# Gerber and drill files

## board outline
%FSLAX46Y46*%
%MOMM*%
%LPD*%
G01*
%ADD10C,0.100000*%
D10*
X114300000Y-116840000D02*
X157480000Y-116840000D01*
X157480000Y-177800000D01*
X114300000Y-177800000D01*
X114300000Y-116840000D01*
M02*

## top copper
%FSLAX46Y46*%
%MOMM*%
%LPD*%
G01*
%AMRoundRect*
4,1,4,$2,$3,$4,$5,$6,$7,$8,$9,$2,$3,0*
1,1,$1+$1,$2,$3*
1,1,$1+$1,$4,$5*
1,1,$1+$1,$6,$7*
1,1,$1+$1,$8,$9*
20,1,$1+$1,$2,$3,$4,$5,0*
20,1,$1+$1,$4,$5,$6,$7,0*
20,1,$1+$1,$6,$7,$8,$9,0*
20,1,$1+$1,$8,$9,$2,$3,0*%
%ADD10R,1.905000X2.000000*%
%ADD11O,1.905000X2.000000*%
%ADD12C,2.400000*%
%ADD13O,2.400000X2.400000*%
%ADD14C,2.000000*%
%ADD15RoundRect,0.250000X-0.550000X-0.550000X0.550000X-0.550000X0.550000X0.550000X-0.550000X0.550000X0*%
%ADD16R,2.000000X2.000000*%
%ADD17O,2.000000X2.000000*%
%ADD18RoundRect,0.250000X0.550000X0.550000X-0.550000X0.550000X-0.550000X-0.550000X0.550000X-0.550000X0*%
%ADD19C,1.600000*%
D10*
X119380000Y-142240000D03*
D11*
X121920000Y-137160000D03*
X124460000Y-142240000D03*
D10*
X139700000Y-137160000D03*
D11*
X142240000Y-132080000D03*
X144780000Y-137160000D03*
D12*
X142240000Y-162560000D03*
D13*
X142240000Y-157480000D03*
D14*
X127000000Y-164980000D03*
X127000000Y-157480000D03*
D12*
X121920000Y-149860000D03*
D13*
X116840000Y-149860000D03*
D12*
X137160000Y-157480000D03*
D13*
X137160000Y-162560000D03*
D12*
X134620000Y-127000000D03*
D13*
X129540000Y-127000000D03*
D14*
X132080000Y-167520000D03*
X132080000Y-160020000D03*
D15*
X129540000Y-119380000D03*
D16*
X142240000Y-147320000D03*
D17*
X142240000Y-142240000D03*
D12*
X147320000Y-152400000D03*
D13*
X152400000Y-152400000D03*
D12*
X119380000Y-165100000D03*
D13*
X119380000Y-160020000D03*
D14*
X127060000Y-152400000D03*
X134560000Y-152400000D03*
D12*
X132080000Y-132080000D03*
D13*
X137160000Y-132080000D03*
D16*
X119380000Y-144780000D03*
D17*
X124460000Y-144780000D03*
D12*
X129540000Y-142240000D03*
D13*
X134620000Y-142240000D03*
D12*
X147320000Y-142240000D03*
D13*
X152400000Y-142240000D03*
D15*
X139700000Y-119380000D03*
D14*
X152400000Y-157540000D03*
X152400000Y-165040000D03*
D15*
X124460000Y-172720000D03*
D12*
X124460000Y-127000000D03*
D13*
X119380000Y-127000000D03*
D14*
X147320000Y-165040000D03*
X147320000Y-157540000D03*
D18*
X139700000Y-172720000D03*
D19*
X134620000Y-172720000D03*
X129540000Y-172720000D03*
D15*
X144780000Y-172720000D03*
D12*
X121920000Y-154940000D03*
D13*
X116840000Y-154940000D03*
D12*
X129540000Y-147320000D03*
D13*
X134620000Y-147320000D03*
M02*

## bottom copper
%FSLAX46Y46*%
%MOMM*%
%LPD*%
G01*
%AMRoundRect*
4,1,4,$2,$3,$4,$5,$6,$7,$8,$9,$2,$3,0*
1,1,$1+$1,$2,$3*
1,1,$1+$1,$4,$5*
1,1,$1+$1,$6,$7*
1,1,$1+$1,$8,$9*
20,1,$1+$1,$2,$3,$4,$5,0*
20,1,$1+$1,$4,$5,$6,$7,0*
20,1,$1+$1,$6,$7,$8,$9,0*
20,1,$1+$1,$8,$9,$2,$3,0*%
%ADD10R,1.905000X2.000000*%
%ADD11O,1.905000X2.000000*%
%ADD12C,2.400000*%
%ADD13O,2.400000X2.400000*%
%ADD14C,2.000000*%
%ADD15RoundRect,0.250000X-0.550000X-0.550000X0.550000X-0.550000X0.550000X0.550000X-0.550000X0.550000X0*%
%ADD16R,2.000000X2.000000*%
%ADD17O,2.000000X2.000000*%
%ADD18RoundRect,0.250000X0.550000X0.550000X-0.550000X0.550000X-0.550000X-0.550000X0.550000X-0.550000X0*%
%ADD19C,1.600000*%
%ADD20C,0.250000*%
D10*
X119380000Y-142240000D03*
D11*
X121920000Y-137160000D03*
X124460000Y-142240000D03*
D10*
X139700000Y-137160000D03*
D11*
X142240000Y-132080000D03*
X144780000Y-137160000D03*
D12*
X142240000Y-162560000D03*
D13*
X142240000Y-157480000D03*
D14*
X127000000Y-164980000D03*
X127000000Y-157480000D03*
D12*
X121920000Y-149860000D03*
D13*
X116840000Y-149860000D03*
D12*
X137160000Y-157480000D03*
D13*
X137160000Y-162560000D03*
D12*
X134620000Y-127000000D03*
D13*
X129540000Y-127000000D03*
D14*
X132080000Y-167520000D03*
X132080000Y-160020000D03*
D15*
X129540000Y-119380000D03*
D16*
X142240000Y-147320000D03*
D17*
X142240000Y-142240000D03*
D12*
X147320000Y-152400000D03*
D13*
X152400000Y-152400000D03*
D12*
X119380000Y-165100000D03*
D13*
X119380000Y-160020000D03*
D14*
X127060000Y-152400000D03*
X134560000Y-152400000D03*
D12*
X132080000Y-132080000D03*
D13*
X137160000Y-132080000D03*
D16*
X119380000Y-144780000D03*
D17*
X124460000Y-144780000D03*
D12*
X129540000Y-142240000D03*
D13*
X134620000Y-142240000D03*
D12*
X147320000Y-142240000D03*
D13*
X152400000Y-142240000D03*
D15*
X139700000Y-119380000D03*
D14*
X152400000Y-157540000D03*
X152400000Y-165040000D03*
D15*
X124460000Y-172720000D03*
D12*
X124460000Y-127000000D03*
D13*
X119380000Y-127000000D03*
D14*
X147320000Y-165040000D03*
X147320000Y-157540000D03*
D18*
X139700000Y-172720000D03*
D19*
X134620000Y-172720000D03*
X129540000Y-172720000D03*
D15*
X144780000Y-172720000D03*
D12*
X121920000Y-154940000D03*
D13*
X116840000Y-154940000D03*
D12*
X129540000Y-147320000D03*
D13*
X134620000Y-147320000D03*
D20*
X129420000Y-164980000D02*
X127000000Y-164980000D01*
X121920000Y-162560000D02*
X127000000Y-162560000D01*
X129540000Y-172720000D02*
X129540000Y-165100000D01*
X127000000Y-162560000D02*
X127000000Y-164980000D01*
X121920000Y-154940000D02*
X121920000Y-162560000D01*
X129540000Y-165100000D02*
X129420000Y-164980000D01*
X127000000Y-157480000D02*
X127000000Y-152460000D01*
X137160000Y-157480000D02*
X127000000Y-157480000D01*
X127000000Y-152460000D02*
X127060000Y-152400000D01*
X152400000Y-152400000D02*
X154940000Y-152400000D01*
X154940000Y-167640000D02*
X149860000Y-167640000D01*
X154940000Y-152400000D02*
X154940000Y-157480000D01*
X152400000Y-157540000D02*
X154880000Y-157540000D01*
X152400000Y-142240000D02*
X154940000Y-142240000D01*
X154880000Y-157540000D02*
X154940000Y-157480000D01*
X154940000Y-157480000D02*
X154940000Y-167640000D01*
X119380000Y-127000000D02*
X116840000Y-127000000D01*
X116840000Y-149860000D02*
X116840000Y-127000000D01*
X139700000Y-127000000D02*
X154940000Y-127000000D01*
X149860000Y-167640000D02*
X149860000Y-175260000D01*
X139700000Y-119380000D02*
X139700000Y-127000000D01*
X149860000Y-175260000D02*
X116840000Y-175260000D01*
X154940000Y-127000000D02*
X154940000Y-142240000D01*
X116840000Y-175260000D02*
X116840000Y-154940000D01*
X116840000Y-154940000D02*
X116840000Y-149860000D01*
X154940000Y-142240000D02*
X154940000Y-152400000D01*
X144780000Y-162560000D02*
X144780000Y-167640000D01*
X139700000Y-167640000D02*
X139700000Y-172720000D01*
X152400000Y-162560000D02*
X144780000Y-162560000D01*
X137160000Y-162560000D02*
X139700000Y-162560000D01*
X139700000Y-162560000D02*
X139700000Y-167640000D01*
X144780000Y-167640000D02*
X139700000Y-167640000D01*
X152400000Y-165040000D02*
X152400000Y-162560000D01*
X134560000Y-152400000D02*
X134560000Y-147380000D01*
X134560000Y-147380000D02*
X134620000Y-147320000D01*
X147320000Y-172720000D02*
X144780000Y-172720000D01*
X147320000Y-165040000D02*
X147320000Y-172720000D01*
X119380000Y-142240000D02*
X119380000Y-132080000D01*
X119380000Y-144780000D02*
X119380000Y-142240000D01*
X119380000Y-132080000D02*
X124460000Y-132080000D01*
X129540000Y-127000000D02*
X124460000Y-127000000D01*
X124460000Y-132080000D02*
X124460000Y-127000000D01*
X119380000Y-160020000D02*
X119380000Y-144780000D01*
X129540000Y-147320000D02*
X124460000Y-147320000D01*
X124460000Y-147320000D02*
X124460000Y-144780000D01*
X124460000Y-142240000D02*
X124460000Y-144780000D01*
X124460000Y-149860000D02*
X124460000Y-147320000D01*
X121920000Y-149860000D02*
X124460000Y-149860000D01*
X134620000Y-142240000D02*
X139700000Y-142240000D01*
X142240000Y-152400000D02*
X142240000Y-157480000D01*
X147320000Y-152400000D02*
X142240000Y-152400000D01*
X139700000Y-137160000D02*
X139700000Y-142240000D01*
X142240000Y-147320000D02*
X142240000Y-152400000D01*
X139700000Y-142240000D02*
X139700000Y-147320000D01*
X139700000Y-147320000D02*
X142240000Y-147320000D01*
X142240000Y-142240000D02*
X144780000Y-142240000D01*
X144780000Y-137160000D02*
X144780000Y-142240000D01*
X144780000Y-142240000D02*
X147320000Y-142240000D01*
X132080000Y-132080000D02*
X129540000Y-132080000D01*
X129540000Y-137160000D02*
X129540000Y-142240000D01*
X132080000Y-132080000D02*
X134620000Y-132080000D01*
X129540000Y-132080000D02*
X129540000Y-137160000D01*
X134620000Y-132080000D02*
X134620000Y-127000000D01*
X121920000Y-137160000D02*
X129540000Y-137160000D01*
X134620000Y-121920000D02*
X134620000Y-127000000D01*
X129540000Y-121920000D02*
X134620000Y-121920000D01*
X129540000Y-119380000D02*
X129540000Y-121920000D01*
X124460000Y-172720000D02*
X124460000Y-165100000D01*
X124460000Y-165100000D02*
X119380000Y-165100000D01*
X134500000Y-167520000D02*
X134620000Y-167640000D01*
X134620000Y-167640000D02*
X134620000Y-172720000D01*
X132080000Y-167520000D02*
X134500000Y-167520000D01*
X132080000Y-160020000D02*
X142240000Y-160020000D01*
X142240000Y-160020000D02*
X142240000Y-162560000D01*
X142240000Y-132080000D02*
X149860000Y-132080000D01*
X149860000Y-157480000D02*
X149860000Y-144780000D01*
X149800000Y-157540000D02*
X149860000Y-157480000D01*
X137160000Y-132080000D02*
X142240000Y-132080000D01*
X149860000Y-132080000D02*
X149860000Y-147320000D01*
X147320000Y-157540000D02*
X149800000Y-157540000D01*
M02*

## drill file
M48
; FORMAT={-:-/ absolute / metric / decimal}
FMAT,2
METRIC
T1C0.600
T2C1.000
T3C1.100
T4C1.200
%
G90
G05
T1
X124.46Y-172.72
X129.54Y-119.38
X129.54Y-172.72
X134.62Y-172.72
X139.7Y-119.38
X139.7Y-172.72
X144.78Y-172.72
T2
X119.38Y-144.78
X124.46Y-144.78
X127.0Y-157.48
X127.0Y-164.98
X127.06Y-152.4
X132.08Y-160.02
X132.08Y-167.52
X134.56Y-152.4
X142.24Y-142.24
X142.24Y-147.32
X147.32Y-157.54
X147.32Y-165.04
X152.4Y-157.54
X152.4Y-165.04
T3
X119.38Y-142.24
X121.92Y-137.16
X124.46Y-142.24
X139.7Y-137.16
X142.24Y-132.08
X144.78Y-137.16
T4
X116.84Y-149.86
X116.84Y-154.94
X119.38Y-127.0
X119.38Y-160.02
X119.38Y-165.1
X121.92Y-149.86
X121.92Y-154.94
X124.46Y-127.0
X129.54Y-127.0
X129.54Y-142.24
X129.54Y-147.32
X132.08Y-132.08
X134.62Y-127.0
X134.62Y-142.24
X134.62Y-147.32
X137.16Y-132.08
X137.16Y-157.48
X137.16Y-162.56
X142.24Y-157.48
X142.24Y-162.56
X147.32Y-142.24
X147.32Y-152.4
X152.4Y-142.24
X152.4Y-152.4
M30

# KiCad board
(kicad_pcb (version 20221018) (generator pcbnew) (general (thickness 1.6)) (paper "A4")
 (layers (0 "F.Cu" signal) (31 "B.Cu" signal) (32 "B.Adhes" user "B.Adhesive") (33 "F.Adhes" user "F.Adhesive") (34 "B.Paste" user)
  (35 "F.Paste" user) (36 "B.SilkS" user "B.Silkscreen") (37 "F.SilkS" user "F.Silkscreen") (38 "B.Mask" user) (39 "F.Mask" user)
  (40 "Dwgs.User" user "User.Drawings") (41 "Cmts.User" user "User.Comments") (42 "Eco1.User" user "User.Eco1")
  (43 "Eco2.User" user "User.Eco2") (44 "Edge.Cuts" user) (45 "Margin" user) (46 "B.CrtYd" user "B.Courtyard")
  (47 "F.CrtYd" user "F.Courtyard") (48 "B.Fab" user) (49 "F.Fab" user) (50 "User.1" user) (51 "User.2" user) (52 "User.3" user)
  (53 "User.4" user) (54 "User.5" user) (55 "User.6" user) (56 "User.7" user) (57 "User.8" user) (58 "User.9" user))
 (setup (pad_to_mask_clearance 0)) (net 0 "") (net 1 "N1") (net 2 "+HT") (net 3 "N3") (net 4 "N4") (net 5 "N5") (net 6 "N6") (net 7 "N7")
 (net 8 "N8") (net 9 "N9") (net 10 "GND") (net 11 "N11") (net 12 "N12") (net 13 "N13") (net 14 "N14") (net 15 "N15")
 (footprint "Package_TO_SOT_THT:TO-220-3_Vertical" (layer "F.Cu") (at 119.38 137.16)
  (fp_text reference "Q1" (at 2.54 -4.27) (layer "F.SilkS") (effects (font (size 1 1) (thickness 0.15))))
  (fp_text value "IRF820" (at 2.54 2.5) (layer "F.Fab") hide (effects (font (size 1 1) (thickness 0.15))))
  (pad "1" thru_hole rect (at 0 5.08) (size 1.905 2) (drill 1.1) (layers "*.Cu" "*.Mask") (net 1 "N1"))
  (pad "2" thru_hole oval (at 2.54 0) (size 1.905 2) (drill 1.1) (layers "*.Cu" "*.Mask") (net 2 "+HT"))
  (pad "3" thru_hole oval (at 5.08 5.08) (size 1.905 2) (drill 1.1) (layers "*.Cu" "*.Mask") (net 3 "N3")))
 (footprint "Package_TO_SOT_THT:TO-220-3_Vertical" (layer "F.Cu") (at 139.7 137.16)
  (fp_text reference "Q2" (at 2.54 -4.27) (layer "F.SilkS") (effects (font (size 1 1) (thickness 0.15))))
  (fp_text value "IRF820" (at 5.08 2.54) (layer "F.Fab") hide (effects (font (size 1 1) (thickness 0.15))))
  (pad "1" thru_hole rect (at 0 0) (size 1.905 2) (drill 1.1) (layers "*.Cu" "*.Mask") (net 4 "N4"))
  (pad "2" thru_hole oval (at 2.54 -5.08) (size 1.905 2) (drill 1.1) (layers "*.Cu" "*.Mask") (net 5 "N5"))
  (pad "3" thru_hole oval (at 5.08 0) (size 1.905 2) (drill 1.1) (layers "*.Cu" "*.Mask") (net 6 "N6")))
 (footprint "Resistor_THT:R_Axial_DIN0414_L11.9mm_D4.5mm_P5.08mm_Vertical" (layer "F.Cu") (at 142.24 162.56 90)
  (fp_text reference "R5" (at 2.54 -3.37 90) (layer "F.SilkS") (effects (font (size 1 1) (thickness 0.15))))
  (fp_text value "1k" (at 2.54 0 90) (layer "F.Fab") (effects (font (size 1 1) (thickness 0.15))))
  (pad "1" thru_hole circle (at 0 0 90) (size 2.4 2.4) (drill 1.2) (layers "*.Cu" "*.Mask") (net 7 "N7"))
  (pad "2" thru_hole oval (at 5.08 0 90) (size 2.4 2.4) (drill 1.2) (layers "*.Cu" "*.Mask") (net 4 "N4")))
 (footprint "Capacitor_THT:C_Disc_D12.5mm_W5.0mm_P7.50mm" (layer "F.Cu") (at 127 164.98 90)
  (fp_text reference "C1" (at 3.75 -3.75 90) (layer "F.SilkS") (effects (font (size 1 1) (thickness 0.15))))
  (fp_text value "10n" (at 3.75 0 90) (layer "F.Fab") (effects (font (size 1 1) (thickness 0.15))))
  (pad "1" thru_hole circle (at 0 0 90) (size 2 2) (drill 1) (layers "*.Cu" "*.Mask") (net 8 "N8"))
  (pad "2" thru_hole circle (at 7.5 0 90) (size 2 2) (drill 1) (layers "*.Cu" "*.Mask") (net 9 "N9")))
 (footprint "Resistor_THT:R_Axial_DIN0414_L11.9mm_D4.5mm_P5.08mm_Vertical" (layer "F.Cu") (at 121.92 149.86 180)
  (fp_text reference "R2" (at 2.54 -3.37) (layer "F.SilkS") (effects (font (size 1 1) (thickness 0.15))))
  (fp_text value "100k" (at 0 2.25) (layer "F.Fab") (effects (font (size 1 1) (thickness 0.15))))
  (pad "1" thru_hole circle (at 0 0 180) (size 2.4 2.4) (drill 1.2) (layers "*.Cu" "*.Mask") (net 3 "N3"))
  (pad "2" thru_hole oval (at 5.08 0 180) (size 2.4 2.4) (drill 1.2) (layers "*.Cu" "*.Mask") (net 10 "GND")))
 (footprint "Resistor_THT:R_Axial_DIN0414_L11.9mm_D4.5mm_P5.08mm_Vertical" (layer "F.Cu") (at 137.16 157.48 -90)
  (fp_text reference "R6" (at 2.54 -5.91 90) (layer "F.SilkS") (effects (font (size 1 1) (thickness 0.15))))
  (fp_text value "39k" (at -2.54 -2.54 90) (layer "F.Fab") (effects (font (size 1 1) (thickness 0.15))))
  (pad "1" thru_hole circle (at 0 0 270) (size 2.4 2.4) (drill 1.2) (layers "*.Cu" "*.Mask") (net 9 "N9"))
  (pad "2" thru_hole oval (at 5.08 0 270) (size 2.4 2.4) (drill 1.2) (layers "*.Cu" "*.Mask") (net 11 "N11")))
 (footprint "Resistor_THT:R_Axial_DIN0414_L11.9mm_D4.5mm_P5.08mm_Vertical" (layer "F.Cu") (at 134.62 127 180)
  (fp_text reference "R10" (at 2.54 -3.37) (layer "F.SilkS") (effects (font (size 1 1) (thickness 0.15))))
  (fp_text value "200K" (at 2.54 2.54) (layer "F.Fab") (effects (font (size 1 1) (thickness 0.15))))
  (pad "1" thru_hole circle (at 0 0 180) (size 2.4 2.4) (drill 1.2) (layers "*.Cu" "*.Mask") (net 2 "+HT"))
  (pad "2" thru_hole oval (at 5.08 0 180) (size 2.4 2.4) (drill 1.2) (layers "*.Cu" "*.Mask") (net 1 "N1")))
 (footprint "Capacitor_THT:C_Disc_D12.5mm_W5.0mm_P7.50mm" (layer "F.Cu") (at 132.08 167.52 90)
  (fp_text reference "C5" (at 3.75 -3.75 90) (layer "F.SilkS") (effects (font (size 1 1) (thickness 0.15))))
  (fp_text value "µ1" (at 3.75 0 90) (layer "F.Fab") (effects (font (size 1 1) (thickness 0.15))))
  (pad "1" thru_hole circle (at 0 0 90) (size 2 2) (drill 1) (layers "*.Cu" "*.Mask") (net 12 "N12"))
  (pad "2" thru_hole circle (at 7.5 0 90) (size 2 2) (drill 1) (layers "*.Cu" "*.Mask") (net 7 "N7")))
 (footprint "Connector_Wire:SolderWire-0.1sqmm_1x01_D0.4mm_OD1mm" (layer "F.Cu") (at 129.54 119.38)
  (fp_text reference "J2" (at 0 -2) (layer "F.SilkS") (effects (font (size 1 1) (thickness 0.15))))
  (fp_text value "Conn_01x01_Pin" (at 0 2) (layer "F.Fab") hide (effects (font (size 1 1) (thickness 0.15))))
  (pad "1" thru_hole roundrect (at 0 0) (size 1.6 1.6) (drill 0.6) (layers "*.Cu" "*.Mask") (roundrect_rratio 0.15625) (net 2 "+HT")))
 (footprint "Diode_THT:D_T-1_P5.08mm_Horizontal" (layer "F.Cu") (at 142.24 147.32 90)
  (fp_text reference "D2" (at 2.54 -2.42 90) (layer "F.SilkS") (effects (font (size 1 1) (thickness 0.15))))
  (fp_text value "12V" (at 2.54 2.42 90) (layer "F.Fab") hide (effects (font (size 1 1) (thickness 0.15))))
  (pad "1" thru_hole rect (at 0 0 90) (size 2 2) (drill 1) (layers "*.Cu" "*.Mask") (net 4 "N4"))
  (pad "2" thru_hole oval (at 5.08 0 90) (size 2 2) (drill 1) (layers "*.Cu" "*.Mask") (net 6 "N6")))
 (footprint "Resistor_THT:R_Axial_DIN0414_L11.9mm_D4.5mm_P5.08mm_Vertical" (layer "F.Cu") (at 147.32 152.4)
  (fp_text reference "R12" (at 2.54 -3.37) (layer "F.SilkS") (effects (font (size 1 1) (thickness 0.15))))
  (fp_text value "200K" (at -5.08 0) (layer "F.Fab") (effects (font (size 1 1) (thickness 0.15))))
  (pad "1" thru_hole circle (at 0 0) (size 2.4 2.4) (drill 1.2) (layers "*.Cu" "*.Mask") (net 4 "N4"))
  (pad "2" thru_hole oval (at 5.08 0) (size 2.4 2.4) (drill 1.2) (layers "*.Cu" "*.Mask") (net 10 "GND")))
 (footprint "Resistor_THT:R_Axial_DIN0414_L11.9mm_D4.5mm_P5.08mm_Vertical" (layer "F.Cu") (at 119.38 165.1 90)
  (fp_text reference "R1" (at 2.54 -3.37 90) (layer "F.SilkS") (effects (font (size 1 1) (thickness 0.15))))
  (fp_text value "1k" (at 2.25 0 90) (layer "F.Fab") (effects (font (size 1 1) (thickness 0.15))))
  (pad "1" thru_hole circle (at 0 0 90) (size 2.4 2.4) (drill 1.2) (layers "*.Cu" "*.Mask") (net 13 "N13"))
  (pad "2" thru_hole oval (at 5.08 0 90) (size 2.4 2.4) (drill 1.2) (layers "*.Cu" "*.Mask") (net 1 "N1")))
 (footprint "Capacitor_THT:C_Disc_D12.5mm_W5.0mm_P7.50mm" (layer "F.Cu") (at 127.06 152.4)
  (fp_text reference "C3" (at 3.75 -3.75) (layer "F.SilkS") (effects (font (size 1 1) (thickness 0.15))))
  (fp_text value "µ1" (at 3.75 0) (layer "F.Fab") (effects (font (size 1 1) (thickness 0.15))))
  (pad "1" thru_hole circle (at 0 0) (size 2 2) (drill 1) (layers "*.Cu" "*.Mask") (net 9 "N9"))
  (pad "2" thru_hole circle (at 7.5 0) (size 2 2) (drill 1) (layers "*.Cu" "*.Mask") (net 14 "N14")))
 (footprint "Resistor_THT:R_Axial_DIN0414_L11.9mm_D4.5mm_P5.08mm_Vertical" (layer "F.Cu") (at 132.08 132.08)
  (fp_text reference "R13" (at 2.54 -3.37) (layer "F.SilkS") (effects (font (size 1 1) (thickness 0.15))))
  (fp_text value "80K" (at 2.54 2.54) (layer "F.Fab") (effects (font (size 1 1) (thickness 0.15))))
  (pad "1" thru_hole circle (at 0 0) (size 2.4 2.4) (drill 1.2) (layers "*.Cu" "*.Mask") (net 2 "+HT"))
  (pad "2" thru_hole oval (at 5.08 0) (size 2.4 2.4) (drill 1.2) (layers "*.Cu" "*.Mask") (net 5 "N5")))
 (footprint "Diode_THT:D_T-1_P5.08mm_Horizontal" (layer "F.Cu") (at 119.38 144.78)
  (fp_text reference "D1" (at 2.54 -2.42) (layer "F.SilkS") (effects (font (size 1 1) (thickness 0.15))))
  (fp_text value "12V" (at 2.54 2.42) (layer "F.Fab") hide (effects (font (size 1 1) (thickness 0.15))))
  (pad "1" thru_hole rect (at 0 0) (size 2 2) (drill 1) (layers "*.Cu" "*.Mask") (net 1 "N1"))
  (pad "2" thru_hole oval (at 5.08 0) (size 2 2) (drill 1) (layers "*.Cu" "*.Mask") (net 3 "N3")))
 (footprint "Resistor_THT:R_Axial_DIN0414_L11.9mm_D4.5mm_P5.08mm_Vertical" (layer "F.Cu") (at 129.54 142.24)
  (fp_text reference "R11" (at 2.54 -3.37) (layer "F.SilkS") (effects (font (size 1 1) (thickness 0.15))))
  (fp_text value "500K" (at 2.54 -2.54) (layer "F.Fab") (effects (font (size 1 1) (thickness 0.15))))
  (pad "1" thru_hole circle (at 0 0) (size 2.4 2.4) (drill 1.2) (layers "*.Cu" "*.Mask") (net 2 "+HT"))
  (pad "2" thru_hole oval (at 5.08 0) (size 2.4 2.4) (drill 1.2) (layers "*.Cu" "*.Mask") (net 4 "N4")))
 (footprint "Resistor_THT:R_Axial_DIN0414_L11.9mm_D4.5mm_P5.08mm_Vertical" (layer "F.Cu") (at 147.32 142.24)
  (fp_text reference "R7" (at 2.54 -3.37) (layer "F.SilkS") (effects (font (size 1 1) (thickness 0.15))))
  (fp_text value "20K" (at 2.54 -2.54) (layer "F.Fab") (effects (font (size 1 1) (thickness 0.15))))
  (pad "1" thru_hole circle (at 0 0) (size 2.4 2.4) (drill 1.2) (layers "*.Cu" "*.Mask") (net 6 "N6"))
  (pad "2" thru_hole oval (at 5.08 0) (size 2.4 2.4) (drill 1.2) (layers "*.Cu" "*.Mask") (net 10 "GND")))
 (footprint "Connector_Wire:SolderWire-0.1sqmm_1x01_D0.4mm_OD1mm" (layer "F.Cu") (at 139.7 119.38)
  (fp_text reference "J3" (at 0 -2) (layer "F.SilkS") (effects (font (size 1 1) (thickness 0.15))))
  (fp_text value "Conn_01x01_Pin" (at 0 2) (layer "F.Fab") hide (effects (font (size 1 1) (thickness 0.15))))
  (pad "1" thru_hole roundrect (at 0 0) (size 1.6 1.6) (drill 0.6) (layers "*.Cu" "*.Mask") (roundrect_rratio 0.15625) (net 10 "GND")))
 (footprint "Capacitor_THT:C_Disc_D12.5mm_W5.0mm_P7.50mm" (layer "F.Cu") (at 152.4 157.54 -90)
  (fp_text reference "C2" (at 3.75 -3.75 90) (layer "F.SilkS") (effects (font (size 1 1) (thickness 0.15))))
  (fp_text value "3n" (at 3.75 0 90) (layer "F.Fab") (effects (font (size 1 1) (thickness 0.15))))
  (pad "1" thru_hole circle (at 0 0 270) (size 2 2) (drill 1) (layers "*.Cu" "*.Mask") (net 10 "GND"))
  (pad "2" thru_hole circle (at 7.5 0 270) (size 2 2) (drill 1) (layers "*.Cu" "*.Mask") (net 11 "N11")))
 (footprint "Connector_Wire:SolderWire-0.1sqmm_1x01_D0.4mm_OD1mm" (layer "F.Cu") (at 124.46 172.72)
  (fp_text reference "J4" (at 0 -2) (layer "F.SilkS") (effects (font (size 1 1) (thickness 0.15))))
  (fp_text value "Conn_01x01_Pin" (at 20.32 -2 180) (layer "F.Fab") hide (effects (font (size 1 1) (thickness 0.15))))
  (pad "1" thru_hole roundrect (at 0 0) (size 1.6 1.6) (drill 0.6) (layers "*.Cu" "*.Mask") (roundrect_rratio 0.15625) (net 13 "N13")))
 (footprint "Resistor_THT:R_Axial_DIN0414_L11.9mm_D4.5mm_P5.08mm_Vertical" (layer "F.Cu") (at 124.46 127 180)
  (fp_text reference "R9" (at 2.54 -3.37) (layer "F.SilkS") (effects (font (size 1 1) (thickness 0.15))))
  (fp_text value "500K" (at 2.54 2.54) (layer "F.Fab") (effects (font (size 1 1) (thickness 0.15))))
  (pad "1" thru_hole circle (at 0 0 180) (size 2.4 2.4) (drill 1.2) (layers "*.Cu" "*.Mask") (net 1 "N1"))
  (pad "2" thru_hole oval (at 5.08 0 180) (size 2.4 2.4) (drill 1.2) (layers "*.Cu" "*.Mask") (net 10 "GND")))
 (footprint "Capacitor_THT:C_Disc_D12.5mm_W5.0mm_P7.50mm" (layer "F.Cu") (at 147.32 165.04 90)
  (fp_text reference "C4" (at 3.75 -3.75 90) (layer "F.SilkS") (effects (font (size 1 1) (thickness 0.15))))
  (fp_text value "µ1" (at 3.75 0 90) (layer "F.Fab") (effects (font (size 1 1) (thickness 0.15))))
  (pad "1" thru_hole circle (at 0 0 90) (size 2 2) (drill 1) (layers "*.Cu" "*.Mask") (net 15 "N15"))
  (pad "2" thru_hole circle (at 7.5 0 90) (size 2 2) (drill 1) (layers "*.Cu" "*.Mask") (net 5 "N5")))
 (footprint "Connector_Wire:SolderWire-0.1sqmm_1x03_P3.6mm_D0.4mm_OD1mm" (layer "F.Cu") (at 139.7 172.72 180)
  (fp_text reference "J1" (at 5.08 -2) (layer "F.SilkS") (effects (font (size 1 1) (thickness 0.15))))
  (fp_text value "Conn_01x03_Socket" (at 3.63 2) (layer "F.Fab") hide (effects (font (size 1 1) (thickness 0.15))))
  (pad "1" thru_hole roundrect (at 0 0 180) (size 1.6 1.6) (drill 0.6) (layers "*.Cu" "*.Mask") (roundrect_rratio 0.15625) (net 11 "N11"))
  (pad "2" thru_hole circle (at 5.08 0 180) (size 1.6 1.6) (drill 0.6) (layers "*.Cu" "*.Mask") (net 12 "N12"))
  (pad "3" thru_hole circle (at 10.16 0 180) (size 1.6 1.6) (drill 0.6) (layers "*.Cu" "*.Mask") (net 8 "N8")))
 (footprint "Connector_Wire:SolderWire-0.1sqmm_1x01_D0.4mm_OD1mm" (layer "F.Cu") (at 144.78 172.72)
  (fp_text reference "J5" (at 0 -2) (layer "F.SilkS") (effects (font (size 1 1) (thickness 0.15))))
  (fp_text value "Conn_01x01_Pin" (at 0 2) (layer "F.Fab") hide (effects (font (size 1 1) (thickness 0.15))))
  (pad "1" thru_hole roundrect (at 0 0) (size 1.6 1.6) (drill 0.6) (layers "*.Cu" "*.Mask") (roundrect_rratio 0.15625) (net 15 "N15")))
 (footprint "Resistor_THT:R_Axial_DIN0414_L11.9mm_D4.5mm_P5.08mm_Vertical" (layer "F.Cu") (at 121.92 154.94 180)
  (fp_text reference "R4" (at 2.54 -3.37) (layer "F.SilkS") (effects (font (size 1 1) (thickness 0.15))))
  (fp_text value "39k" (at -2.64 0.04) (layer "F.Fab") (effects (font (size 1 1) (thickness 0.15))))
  (pad "1" thru_hole circle (at 0 0 180) (size 2.4 2.4) (drill 1.2) (layers "*.Cu" "*.Mask") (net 8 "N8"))
  (pad "2" thru_hole oval (at 5.08 0 180) (size 2.4 2.4) (drill 1.2) (layers "*.Cu" "*.Mask") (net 10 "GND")))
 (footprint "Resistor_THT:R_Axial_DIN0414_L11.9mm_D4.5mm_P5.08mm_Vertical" (layer "F.Cu") (at 129.54 147.32)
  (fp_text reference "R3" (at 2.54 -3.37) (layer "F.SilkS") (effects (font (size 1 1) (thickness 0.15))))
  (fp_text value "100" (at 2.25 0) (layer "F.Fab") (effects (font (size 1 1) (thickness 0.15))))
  (pad "1" thru_hole circle (at 0 0) (size 2.4 2.4) (drill 1.2) (layers "*.Cu" "*.Mask") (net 3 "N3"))
  (pad "2" thru_hole oval (at 5.08 0) (size 2.4 2.4) (drill 1.2) (layers "*.Cu" "*.Mask") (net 14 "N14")))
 (gr_rect (start 114.3 116.84) (end 157.48 177.8) (stroke (width 0.1) (type default)) (fill none) (layer "Edge.Cuts"))
 (segment (start 129.42 164.98) (end 127 164.98) (width 0.25) (layer "B.Cu") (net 8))
 (segment (start 121.92 162.56) (end 127 162.56) (width 0.25) (layer "B.Cu") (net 8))
 (segment (start 129.54 172.72) (end 129.54 165.1) (width 0.25) (layer "B.Cu") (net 8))
 (segment (start 127 162.56) (end 127 164.98) (width 0.25) (layer "B.Cu") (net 8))
 (segment (start 121.92 154.94) (end 121.92 162.56) (width 0.25) (layer "B.Cu") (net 8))
 (segment (start 129.54 165.1) (end 129.42 164.98) (width 0.25) (layer "B.Cu") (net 8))
 (segment (start 127 157.48) (end 127 152.46) (width 0.25) (layer "B.Cu") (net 9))
 (segment (start 137.16 157.48) (end 127 157.48) (width 0.25) (layer "B.Cu") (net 9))
 (segment (start 127 152.46) (end 127.06 152.4) (width 0.25) (layer "B.Cu") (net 9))
 (segment (start 152.4 152.4) (end 154.94 152.4) (width 0.25) (layer "B.Cu") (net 10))
 (segment (start 154.94 167.64) (end 149.86 167.64) (width 0.25) (layer "B.Cu") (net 10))
 (segment (start 154.94 152.4) (end 154.94 157.48) (width 0.25) (layer "B.Cu") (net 10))
 (segment (start 152.4 157.54) (end 154.88 157.54) (width 0.25) (layer "B.Cu") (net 10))
 (segment (start 152.4 142.24) (end 154.94 142.24) (width 0.25) (layer "B.Cu") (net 10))
 (segment (start 154.88 157.54) (end 154.94 157.48) (width 0.25) (layer "B.Cu") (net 10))
 (segment (start 154.94 157.48) (end 154.94 167.64) (width 0.25) (layer "B.Cu") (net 10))
 (segment (start 119.38 127) (end 116.84 127) (width 0.25) (layer "B.Cu") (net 10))
 (segment (start 116.84 149.86) (end 116.84 127) (width 0.25) (layer "B.Cu") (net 10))
 (segment (start 139.7 127) (end 154.94 127) (width 0.25) (layer "B.Cu") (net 10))
 (segment (start 149.86 167.64) (end 149.86 175.26) (width 0.25) (layer "B.Cu") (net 10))
 (segment (start 139.7 119.38) (end 139.7 127) (width 0.25) (layer "B.Cu") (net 10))
 (segment (start 149.86 175.26) (end 116.84 175.26) (width 0.25) (layer "B.Cu") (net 10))
 (segment (start 154.94 127) (end 154.94 142.24) (width 0.25) (layer "B.Cu") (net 10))
 (segment (start 116.84 175.26) (end 116.84 154.94) (width 0.25) (layer "B.Cu") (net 10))
 (segment (start 116.84 154.94) (end 116.84 149.86) (width 0.25) (layer "B.Cu") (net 10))
 (segment (start 154.94 142.24) (end 154.94 152.4) (width 0.25) (layer "B.Cu") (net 10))
 (segment (start 144.78 162.56) (end 144.78 167.64) (width 0.25) (layer "B.Cu") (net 11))
 (segment (start 139.7 167.64) (end 139.7 172.72) (width 0.25) (layer "B.Cu") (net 11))
 (segment (start 152.4 162.56) (end 144.78 162.56) (width 0.25) (layer "B.Cu") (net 11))
 (segment (start 137.16 162.56) (end 139.7 162.56) (width 0.25) (layer "B.Cu") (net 11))
 (segment (start 139.7 162.56) (end 139.7 167.64) (width 0.25) (layer "B.Cu") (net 11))
 (segment (start 144.78 167.64) (end 139.7 167.64) (width 0.25) (layer "B.Cu") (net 11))
 (segment (start 152.4 165.04) (end 152.4 162.56) (width 0.25) (layer "B.Cu") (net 11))
 (segment (start 134.56 152.4) (end 134.56 147.38) (width 0.25) (layer "B.Cu") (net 14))
 (segment (start 134.56 147.38) (end 134.62 147.32) (width 0.25) (layer "B.Cu") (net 14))
 (segment (start 147.32 172.72) (end 144.78 172.72) (width 0.25) (layer "B.Cu") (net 15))
 (segment (start 147.32 165.04) (end 147.32 172.72) (width 0.25) (layer "B.Cu") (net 15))
 (segment (start 119.38 142.24) (end 119.38 132.08) (width 0.25) (layer "B.Cu") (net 1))
 (segment (start 119.38 144.78) (end 119.38 142.24) (width 0.25) (layer "B.Cu") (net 1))
 (segment (start 119.38 132.08) (end 124.46 132.08) (width 0.25) (layer "B.Cu") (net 1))
 (segment (start 129.54 127) (end 124.46 127) (width 0.25) (layer "B.Cu") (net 1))
 (segment (start 124.46 132.08) (end 124.46 127) (width 0.25) (layer "B.Cu") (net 1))
 (segment (start 119.38 160.02) (end 119.38 144.78) (width 0.25) (layer "B.Cu") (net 1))
 (segment (start 129.54 147.32) (end 124.46 147.32) (width 0.25) (layer "B.Cu") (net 3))
 (segment (start 124.46 147.32) (end 124.46 144.78) (width 0.25) (layer "B.Cu") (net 3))
 (segment (start 124.46 142.24) (end 124.46 144.78) (width 0.25) (layer "B.Cu") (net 3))
 (segment (start 124.46 149.86) (end 124.46 147.32) (width 0.25) (layer "B.Cu") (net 3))
 (segment (start 121.92 149.86) (end 124.46 149.86) (width 0.25) (layer "B.Cu") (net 3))
 (segment (start 134.62 142.24) (end 139.7 142.24) (width 0.25) (layer "B.Cu") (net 4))
 (segment (start 142.24 152.4) (end 142.24 157.48) (width 0.25) (layer "B.Cu") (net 4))
 (segment (start 147.32 152.4) (end 142.24 152.4) (width 0.25) (layer "B.Cu") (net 4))
 (segment (start 139.7 137.16) (end 139.7 142.24) (width 0.25) (layer "B.Cu") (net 4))
 (segment (start 142.24 147.32) (end 142.24 152.4) (width 0.25) (layer "B.Cu") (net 4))
 (segment (start 139.7 142.24) (end 139.7 147.32) (width 0.25) (layer "B.Cu") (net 4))
 (segment (start 139.7 147.32) (end 142.24 147.32) (width 0.25) (layer "B.Cu") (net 4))
 (segment (start 142.24 142.24) (end 144.78 142.24) (width 0.25) (layer "B.Cu") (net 6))
 (segment (start 144.78 137.16) (end 144.78 142.24) (width 0.25) (layer "B.Cu") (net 6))
 (segment (start 144.78 142.24) (end 147.32 142.24) (width 0.25) (layer "B.Cu") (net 6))
 (segment (start 132.08 132.08) (end 129.54 132.08) (width 0.25) (layer "B.Cu") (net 2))
 (segment (start 129.54 137.16) (end 129.54 142.24) (width 0.25) (layer "B.Cu") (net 2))
 (segment (start 132.08 132.08) (end 134.62 132.08) (width 0.25) (layer "B.Cu") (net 2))
 (segment (start 129.54 132.08) (end 129.54 137.16) (width 0.25) (layer "B.Cu") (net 2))
 (segment (start 134.62 132.08) (end 134.62 127) (width 0.25) (layer "B.Cu") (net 2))
 (segment (start 121.92 137.16) (end 129.54 137.16) (width 0.25) (layer "B.Cu") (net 2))
 (segment (start 134.62 121.92) (end 134.62 127) (width 0.25) (layer "B.Cu") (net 2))
 (segment (start 129.54 121.92) (end 134.62 121.92) (width 0.25) (layer "B.Cu") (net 2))
 (segment (start 129.54 119.38) (end 129.54 121.92) (width 0.25) (layer "B.Cu") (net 2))
 (segment (start 124.46 172.72) (end 124.46 165.1) (width 0.25) (layer "B.Cu") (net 13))
 (segment (start 124.46 165.1) (end 119.38 165.1) (width 0.25) (layer "B.Cu") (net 13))
 (segment (start 134.5 167.52) (end 134.62 167.64) (width 0.25) (layer "B.Cu") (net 12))
 (segment (start 134.62 167.64) (end 134.62 172.72) (width 0.25) (layer "B.Cu") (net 12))
 (segment (start 132.08 167.52) (end 134.5 167.52) (width 0.25) (layer "B.Cu") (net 12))
 (segment (start 132.08 160.02) (end 142.24 160.02) (width 0.25) (layer "B.Cu") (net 7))
 (segment (start 142.24 160.02) (end 142.24 162.56) (width 0.25) (layer "B.Cu") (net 7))
 (segment (start 142.24 132.08) (end 149.86 132.08) (width 0.25) (layer "B.Cu") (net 5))
 (segment (start 149.86 157.48) (end 149.86 144.78) (width 0.25) (layer "B.Cu") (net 5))
 (segment (start 149.8 157.54) (end 149.86 157.48) (width 0.25) (layer "B.Cu") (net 5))
 (segment (start 137.16 132.08) (end 142.24 132.08) (width 0.25) (layer "B.Cu") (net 5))
 (segment (start 149.86 132.08) (end 149.86 147.32) (width 0.25) (layer "B.Cu") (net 5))
 (segment (start 147.32 157.54) (end 149.8 157.54) (width 0.25) (layer "B.Cu") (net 5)))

